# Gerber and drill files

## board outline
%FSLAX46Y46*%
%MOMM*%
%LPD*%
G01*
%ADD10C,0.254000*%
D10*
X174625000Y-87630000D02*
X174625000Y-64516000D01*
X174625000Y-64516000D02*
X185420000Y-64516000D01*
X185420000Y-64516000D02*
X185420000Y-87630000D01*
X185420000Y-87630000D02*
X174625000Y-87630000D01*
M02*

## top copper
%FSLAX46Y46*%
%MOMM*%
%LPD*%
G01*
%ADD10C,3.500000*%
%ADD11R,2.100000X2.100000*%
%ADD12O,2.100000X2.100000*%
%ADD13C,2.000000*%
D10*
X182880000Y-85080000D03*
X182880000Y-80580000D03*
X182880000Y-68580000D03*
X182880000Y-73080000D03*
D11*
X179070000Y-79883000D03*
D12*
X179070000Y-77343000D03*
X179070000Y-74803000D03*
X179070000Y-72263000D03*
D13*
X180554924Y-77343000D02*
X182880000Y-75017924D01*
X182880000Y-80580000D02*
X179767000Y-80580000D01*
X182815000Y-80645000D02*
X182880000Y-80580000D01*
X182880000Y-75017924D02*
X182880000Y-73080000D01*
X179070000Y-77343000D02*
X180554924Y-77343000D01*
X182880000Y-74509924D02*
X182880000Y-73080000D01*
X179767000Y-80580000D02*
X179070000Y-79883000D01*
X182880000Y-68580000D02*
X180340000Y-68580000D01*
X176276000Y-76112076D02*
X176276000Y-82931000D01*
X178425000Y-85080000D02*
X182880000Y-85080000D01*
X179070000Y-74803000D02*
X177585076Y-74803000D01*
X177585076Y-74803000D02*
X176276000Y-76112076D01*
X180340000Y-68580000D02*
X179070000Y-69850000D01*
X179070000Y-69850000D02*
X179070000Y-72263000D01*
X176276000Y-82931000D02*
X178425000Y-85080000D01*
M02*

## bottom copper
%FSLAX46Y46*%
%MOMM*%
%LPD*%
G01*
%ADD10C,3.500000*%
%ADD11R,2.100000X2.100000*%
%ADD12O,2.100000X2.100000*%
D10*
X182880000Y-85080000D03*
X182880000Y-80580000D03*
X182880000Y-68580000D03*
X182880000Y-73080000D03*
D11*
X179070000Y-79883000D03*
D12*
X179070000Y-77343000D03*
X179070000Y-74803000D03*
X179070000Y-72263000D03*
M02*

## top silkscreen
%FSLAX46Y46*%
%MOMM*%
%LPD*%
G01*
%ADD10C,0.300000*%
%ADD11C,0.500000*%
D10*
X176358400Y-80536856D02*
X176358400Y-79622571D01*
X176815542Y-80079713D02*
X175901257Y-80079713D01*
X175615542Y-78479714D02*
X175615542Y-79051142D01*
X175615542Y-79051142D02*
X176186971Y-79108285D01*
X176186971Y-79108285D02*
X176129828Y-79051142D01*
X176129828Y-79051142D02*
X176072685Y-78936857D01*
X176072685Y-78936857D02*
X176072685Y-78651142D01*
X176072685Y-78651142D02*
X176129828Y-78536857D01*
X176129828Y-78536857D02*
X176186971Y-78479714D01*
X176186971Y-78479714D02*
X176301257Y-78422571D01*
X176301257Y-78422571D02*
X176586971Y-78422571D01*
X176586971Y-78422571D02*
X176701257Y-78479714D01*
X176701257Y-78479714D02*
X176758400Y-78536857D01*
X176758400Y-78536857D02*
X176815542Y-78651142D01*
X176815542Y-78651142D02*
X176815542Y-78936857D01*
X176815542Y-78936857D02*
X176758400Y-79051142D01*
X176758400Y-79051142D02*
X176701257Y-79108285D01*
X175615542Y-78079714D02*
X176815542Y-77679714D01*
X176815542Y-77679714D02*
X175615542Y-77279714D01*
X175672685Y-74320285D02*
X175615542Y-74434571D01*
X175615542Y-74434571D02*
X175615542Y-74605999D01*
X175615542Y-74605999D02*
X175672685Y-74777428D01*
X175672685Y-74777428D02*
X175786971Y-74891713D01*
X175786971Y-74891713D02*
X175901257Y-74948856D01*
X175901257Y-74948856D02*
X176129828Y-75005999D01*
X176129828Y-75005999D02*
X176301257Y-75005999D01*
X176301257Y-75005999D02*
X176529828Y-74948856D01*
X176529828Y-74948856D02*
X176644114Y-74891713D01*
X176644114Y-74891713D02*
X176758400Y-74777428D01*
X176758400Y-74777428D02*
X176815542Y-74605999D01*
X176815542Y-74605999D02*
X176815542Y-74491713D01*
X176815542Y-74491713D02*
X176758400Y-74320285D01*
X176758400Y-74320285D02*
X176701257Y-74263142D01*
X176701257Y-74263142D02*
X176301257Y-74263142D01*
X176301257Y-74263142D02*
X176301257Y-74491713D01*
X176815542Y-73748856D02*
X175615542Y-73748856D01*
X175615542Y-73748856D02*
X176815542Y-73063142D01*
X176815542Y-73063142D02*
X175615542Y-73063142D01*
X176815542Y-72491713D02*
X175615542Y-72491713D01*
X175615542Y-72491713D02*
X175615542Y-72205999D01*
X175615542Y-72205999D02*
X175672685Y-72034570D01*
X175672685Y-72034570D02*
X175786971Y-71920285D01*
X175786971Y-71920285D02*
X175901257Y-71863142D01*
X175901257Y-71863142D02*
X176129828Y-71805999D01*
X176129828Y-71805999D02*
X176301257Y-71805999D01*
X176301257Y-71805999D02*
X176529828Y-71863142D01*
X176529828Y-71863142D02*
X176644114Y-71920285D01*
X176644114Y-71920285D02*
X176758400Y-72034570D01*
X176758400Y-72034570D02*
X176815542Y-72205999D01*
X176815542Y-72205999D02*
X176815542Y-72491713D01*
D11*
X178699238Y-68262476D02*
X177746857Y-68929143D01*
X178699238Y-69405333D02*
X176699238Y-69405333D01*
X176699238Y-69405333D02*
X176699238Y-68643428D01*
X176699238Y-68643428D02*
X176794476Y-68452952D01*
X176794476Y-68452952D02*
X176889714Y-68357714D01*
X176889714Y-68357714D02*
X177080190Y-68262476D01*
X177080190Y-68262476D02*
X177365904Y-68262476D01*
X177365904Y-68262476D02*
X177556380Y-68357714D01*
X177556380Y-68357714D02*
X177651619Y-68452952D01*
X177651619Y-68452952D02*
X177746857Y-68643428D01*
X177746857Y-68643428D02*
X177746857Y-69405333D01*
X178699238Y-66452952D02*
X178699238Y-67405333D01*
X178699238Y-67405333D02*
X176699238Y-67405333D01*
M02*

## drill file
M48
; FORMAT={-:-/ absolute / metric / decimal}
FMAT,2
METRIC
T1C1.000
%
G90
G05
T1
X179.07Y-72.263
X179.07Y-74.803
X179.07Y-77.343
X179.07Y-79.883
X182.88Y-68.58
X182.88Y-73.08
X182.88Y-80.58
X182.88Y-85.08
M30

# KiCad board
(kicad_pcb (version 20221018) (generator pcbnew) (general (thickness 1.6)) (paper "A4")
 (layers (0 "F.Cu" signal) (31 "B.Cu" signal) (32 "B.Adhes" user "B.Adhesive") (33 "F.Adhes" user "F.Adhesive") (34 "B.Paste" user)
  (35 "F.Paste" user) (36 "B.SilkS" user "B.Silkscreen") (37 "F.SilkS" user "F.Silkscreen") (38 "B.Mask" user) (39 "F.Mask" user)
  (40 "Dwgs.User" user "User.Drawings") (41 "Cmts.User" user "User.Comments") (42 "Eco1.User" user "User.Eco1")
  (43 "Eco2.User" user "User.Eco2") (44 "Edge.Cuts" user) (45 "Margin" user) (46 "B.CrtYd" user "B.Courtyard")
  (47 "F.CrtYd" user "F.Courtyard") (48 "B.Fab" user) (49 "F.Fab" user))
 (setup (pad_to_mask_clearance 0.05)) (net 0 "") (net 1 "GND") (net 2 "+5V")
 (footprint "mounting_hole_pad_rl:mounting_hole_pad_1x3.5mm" (layer "F.Cu") (at 182.88 85.08)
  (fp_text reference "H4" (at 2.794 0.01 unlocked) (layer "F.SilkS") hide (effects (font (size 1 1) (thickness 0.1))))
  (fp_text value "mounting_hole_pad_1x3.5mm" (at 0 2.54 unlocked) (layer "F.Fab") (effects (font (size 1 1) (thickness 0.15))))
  (pad "1" thru_hole circle (at 0 0) (size 3.5 3.5) (drill 1) (layers "*.Cu" "*.Mask") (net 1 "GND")))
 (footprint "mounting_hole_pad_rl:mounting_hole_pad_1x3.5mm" (layer "F.Cu") (at 182.88 80.58)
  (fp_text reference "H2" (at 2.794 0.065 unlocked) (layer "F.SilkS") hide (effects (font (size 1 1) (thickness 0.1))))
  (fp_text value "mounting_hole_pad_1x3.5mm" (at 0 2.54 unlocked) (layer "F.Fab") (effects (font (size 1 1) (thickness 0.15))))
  (pad "1" thru_hole circle (at 0 0) (size 3.5 3.5) (drill 1) (layers "*.Cu" "*.Mask") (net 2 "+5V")))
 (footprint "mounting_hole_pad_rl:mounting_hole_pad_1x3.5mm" (layer "F.Cu") (at 182.88 68.58)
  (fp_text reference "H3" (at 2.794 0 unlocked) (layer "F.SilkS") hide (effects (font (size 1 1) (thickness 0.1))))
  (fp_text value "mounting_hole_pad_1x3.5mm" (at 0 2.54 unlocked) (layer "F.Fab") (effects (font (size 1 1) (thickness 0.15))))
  (pad "1" thru_hole circle (at 0 0) (size 3.5 3.5) (drill 1) (layers "*.Cu" "*.Mask") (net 1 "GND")))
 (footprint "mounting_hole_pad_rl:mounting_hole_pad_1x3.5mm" (layer "F.Cu") (at 182.88 73.08)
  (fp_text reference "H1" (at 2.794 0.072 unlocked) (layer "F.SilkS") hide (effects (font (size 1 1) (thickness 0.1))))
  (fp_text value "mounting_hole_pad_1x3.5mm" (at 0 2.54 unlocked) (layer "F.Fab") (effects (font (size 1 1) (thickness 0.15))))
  (pad "1" thru_hole circle (at 0 0) (size 3.5 3.5) (drill 1) (layers "*.Cu" "*.Mask") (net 2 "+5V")))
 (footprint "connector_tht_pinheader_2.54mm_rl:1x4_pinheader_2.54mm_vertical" (layer "B.Cu") (at 179.07 79.883)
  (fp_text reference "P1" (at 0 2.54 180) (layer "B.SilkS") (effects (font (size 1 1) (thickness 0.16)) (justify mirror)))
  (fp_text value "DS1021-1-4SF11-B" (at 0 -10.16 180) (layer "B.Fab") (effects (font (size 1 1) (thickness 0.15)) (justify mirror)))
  (pad "1" thru_hole rect (at 0 0) (size 2.1 2.1) (drill 1) (layers "*.Cu" "*.Mask") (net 2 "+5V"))
  (pad "2" thru_hole oval (at 0 -2.54) (size 2.1 2.1) (drill 1) (layers "*.Cu" "*.Mask") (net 2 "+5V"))
  (pad "3" thru_hole oval (at 0 -5.08) (size 2.1 2.1) (drill 1) (layers "*.Cu" "*.Mask") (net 1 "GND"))
  (pad "4" thru_hole oval (at 0 -7.62) (size 2.1 2.1) (drill 1) (layers "*.Cu" "*.Mask") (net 1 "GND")))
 (gr_line (start 174.625 87.63) (end 174.625 64.516) (stroke (width 0.254) (type solid)) (layer "Edge.Cuts"))
 (gr_line (start 174.625 64.516) (end 185.42 64.516) (stroke (width 0.254) (type solid)) (layer "Edge.Cuts"))
 (gr_line (start 185.42 64.516) (end 185.42 87.63) (stroke (width 0.254) (type solid)) (layer "Edge.Cuts"))
 (gr_line (start 185.42 87.63) (end 174.625 87.63) (stroke (width 0.254) (type solid)) (layer "Edge.Cuts"))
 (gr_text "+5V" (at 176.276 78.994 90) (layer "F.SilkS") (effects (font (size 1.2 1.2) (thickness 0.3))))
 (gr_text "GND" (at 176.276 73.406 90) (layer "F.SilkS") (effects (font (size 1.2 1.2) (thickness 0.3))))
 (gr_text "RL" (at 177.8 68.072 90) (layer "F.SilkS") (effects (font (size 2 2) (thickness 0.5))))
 (segment (start 180.554924 77.343) (end 182.88 75.017924) (width 2) (layer "F.Cu") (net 2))
 (segment (start 182.88 80.58) (end 179.767 80.58) (width 2) (layer "F.Cu") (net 2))
 (segment (start 182.815 80.645) (end 182.88 80.58) (width 2) (layer "F.Cu") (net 2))
 (segment (start 182.88 75.017924) (end 182.88 73.08) (width 2) (layer "F.Cu") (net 2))
 (segment (start 179.07 77.343) (end 180.554924 77.343) (width 2) (layer "F.Cu") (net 2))
 (segment (start 182.88 74.509924) (end 182.88 73.08) (width 2) (layer "F.Cu") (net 2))
 (segment (start 179.767 80.58) (end 179.07 79.883) (width 2) (layer "F.Cu") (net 2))
 (segment (start 182.88 68.58) (end 180.34 68.58) (width 2) (layer "F.Cu") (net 1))
 (segment (start 176.276 76.112076) (end 176.276 82.931) (width 2) (layer "F.Cu") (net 1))
 (segment (start 178.425 85.08) (end 182.88 85.08) (width 2) (layer "F.Cu") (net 1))
 (segment (start 179.07 74.803) (end 177.585076 74.803) (width 2) (layer "F.Cu") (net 1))
 (segment (start 177.585076 74.803) (end 176.276 76.112076) (width 2) (layer "F.Cu") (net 1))
 (segment (start 180.34 68.58) (end 179.07 69.85) (width 2) (layer "F.Cu") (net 1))
 (segment (start 179.07 69.85) (end 179.07 72.263) (width 2) (layer "F.Cu") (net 1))
 (segment (start 176.276 82.931) (end 178.425 85.08) (width 2) (layer "F.Cu") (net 1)))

